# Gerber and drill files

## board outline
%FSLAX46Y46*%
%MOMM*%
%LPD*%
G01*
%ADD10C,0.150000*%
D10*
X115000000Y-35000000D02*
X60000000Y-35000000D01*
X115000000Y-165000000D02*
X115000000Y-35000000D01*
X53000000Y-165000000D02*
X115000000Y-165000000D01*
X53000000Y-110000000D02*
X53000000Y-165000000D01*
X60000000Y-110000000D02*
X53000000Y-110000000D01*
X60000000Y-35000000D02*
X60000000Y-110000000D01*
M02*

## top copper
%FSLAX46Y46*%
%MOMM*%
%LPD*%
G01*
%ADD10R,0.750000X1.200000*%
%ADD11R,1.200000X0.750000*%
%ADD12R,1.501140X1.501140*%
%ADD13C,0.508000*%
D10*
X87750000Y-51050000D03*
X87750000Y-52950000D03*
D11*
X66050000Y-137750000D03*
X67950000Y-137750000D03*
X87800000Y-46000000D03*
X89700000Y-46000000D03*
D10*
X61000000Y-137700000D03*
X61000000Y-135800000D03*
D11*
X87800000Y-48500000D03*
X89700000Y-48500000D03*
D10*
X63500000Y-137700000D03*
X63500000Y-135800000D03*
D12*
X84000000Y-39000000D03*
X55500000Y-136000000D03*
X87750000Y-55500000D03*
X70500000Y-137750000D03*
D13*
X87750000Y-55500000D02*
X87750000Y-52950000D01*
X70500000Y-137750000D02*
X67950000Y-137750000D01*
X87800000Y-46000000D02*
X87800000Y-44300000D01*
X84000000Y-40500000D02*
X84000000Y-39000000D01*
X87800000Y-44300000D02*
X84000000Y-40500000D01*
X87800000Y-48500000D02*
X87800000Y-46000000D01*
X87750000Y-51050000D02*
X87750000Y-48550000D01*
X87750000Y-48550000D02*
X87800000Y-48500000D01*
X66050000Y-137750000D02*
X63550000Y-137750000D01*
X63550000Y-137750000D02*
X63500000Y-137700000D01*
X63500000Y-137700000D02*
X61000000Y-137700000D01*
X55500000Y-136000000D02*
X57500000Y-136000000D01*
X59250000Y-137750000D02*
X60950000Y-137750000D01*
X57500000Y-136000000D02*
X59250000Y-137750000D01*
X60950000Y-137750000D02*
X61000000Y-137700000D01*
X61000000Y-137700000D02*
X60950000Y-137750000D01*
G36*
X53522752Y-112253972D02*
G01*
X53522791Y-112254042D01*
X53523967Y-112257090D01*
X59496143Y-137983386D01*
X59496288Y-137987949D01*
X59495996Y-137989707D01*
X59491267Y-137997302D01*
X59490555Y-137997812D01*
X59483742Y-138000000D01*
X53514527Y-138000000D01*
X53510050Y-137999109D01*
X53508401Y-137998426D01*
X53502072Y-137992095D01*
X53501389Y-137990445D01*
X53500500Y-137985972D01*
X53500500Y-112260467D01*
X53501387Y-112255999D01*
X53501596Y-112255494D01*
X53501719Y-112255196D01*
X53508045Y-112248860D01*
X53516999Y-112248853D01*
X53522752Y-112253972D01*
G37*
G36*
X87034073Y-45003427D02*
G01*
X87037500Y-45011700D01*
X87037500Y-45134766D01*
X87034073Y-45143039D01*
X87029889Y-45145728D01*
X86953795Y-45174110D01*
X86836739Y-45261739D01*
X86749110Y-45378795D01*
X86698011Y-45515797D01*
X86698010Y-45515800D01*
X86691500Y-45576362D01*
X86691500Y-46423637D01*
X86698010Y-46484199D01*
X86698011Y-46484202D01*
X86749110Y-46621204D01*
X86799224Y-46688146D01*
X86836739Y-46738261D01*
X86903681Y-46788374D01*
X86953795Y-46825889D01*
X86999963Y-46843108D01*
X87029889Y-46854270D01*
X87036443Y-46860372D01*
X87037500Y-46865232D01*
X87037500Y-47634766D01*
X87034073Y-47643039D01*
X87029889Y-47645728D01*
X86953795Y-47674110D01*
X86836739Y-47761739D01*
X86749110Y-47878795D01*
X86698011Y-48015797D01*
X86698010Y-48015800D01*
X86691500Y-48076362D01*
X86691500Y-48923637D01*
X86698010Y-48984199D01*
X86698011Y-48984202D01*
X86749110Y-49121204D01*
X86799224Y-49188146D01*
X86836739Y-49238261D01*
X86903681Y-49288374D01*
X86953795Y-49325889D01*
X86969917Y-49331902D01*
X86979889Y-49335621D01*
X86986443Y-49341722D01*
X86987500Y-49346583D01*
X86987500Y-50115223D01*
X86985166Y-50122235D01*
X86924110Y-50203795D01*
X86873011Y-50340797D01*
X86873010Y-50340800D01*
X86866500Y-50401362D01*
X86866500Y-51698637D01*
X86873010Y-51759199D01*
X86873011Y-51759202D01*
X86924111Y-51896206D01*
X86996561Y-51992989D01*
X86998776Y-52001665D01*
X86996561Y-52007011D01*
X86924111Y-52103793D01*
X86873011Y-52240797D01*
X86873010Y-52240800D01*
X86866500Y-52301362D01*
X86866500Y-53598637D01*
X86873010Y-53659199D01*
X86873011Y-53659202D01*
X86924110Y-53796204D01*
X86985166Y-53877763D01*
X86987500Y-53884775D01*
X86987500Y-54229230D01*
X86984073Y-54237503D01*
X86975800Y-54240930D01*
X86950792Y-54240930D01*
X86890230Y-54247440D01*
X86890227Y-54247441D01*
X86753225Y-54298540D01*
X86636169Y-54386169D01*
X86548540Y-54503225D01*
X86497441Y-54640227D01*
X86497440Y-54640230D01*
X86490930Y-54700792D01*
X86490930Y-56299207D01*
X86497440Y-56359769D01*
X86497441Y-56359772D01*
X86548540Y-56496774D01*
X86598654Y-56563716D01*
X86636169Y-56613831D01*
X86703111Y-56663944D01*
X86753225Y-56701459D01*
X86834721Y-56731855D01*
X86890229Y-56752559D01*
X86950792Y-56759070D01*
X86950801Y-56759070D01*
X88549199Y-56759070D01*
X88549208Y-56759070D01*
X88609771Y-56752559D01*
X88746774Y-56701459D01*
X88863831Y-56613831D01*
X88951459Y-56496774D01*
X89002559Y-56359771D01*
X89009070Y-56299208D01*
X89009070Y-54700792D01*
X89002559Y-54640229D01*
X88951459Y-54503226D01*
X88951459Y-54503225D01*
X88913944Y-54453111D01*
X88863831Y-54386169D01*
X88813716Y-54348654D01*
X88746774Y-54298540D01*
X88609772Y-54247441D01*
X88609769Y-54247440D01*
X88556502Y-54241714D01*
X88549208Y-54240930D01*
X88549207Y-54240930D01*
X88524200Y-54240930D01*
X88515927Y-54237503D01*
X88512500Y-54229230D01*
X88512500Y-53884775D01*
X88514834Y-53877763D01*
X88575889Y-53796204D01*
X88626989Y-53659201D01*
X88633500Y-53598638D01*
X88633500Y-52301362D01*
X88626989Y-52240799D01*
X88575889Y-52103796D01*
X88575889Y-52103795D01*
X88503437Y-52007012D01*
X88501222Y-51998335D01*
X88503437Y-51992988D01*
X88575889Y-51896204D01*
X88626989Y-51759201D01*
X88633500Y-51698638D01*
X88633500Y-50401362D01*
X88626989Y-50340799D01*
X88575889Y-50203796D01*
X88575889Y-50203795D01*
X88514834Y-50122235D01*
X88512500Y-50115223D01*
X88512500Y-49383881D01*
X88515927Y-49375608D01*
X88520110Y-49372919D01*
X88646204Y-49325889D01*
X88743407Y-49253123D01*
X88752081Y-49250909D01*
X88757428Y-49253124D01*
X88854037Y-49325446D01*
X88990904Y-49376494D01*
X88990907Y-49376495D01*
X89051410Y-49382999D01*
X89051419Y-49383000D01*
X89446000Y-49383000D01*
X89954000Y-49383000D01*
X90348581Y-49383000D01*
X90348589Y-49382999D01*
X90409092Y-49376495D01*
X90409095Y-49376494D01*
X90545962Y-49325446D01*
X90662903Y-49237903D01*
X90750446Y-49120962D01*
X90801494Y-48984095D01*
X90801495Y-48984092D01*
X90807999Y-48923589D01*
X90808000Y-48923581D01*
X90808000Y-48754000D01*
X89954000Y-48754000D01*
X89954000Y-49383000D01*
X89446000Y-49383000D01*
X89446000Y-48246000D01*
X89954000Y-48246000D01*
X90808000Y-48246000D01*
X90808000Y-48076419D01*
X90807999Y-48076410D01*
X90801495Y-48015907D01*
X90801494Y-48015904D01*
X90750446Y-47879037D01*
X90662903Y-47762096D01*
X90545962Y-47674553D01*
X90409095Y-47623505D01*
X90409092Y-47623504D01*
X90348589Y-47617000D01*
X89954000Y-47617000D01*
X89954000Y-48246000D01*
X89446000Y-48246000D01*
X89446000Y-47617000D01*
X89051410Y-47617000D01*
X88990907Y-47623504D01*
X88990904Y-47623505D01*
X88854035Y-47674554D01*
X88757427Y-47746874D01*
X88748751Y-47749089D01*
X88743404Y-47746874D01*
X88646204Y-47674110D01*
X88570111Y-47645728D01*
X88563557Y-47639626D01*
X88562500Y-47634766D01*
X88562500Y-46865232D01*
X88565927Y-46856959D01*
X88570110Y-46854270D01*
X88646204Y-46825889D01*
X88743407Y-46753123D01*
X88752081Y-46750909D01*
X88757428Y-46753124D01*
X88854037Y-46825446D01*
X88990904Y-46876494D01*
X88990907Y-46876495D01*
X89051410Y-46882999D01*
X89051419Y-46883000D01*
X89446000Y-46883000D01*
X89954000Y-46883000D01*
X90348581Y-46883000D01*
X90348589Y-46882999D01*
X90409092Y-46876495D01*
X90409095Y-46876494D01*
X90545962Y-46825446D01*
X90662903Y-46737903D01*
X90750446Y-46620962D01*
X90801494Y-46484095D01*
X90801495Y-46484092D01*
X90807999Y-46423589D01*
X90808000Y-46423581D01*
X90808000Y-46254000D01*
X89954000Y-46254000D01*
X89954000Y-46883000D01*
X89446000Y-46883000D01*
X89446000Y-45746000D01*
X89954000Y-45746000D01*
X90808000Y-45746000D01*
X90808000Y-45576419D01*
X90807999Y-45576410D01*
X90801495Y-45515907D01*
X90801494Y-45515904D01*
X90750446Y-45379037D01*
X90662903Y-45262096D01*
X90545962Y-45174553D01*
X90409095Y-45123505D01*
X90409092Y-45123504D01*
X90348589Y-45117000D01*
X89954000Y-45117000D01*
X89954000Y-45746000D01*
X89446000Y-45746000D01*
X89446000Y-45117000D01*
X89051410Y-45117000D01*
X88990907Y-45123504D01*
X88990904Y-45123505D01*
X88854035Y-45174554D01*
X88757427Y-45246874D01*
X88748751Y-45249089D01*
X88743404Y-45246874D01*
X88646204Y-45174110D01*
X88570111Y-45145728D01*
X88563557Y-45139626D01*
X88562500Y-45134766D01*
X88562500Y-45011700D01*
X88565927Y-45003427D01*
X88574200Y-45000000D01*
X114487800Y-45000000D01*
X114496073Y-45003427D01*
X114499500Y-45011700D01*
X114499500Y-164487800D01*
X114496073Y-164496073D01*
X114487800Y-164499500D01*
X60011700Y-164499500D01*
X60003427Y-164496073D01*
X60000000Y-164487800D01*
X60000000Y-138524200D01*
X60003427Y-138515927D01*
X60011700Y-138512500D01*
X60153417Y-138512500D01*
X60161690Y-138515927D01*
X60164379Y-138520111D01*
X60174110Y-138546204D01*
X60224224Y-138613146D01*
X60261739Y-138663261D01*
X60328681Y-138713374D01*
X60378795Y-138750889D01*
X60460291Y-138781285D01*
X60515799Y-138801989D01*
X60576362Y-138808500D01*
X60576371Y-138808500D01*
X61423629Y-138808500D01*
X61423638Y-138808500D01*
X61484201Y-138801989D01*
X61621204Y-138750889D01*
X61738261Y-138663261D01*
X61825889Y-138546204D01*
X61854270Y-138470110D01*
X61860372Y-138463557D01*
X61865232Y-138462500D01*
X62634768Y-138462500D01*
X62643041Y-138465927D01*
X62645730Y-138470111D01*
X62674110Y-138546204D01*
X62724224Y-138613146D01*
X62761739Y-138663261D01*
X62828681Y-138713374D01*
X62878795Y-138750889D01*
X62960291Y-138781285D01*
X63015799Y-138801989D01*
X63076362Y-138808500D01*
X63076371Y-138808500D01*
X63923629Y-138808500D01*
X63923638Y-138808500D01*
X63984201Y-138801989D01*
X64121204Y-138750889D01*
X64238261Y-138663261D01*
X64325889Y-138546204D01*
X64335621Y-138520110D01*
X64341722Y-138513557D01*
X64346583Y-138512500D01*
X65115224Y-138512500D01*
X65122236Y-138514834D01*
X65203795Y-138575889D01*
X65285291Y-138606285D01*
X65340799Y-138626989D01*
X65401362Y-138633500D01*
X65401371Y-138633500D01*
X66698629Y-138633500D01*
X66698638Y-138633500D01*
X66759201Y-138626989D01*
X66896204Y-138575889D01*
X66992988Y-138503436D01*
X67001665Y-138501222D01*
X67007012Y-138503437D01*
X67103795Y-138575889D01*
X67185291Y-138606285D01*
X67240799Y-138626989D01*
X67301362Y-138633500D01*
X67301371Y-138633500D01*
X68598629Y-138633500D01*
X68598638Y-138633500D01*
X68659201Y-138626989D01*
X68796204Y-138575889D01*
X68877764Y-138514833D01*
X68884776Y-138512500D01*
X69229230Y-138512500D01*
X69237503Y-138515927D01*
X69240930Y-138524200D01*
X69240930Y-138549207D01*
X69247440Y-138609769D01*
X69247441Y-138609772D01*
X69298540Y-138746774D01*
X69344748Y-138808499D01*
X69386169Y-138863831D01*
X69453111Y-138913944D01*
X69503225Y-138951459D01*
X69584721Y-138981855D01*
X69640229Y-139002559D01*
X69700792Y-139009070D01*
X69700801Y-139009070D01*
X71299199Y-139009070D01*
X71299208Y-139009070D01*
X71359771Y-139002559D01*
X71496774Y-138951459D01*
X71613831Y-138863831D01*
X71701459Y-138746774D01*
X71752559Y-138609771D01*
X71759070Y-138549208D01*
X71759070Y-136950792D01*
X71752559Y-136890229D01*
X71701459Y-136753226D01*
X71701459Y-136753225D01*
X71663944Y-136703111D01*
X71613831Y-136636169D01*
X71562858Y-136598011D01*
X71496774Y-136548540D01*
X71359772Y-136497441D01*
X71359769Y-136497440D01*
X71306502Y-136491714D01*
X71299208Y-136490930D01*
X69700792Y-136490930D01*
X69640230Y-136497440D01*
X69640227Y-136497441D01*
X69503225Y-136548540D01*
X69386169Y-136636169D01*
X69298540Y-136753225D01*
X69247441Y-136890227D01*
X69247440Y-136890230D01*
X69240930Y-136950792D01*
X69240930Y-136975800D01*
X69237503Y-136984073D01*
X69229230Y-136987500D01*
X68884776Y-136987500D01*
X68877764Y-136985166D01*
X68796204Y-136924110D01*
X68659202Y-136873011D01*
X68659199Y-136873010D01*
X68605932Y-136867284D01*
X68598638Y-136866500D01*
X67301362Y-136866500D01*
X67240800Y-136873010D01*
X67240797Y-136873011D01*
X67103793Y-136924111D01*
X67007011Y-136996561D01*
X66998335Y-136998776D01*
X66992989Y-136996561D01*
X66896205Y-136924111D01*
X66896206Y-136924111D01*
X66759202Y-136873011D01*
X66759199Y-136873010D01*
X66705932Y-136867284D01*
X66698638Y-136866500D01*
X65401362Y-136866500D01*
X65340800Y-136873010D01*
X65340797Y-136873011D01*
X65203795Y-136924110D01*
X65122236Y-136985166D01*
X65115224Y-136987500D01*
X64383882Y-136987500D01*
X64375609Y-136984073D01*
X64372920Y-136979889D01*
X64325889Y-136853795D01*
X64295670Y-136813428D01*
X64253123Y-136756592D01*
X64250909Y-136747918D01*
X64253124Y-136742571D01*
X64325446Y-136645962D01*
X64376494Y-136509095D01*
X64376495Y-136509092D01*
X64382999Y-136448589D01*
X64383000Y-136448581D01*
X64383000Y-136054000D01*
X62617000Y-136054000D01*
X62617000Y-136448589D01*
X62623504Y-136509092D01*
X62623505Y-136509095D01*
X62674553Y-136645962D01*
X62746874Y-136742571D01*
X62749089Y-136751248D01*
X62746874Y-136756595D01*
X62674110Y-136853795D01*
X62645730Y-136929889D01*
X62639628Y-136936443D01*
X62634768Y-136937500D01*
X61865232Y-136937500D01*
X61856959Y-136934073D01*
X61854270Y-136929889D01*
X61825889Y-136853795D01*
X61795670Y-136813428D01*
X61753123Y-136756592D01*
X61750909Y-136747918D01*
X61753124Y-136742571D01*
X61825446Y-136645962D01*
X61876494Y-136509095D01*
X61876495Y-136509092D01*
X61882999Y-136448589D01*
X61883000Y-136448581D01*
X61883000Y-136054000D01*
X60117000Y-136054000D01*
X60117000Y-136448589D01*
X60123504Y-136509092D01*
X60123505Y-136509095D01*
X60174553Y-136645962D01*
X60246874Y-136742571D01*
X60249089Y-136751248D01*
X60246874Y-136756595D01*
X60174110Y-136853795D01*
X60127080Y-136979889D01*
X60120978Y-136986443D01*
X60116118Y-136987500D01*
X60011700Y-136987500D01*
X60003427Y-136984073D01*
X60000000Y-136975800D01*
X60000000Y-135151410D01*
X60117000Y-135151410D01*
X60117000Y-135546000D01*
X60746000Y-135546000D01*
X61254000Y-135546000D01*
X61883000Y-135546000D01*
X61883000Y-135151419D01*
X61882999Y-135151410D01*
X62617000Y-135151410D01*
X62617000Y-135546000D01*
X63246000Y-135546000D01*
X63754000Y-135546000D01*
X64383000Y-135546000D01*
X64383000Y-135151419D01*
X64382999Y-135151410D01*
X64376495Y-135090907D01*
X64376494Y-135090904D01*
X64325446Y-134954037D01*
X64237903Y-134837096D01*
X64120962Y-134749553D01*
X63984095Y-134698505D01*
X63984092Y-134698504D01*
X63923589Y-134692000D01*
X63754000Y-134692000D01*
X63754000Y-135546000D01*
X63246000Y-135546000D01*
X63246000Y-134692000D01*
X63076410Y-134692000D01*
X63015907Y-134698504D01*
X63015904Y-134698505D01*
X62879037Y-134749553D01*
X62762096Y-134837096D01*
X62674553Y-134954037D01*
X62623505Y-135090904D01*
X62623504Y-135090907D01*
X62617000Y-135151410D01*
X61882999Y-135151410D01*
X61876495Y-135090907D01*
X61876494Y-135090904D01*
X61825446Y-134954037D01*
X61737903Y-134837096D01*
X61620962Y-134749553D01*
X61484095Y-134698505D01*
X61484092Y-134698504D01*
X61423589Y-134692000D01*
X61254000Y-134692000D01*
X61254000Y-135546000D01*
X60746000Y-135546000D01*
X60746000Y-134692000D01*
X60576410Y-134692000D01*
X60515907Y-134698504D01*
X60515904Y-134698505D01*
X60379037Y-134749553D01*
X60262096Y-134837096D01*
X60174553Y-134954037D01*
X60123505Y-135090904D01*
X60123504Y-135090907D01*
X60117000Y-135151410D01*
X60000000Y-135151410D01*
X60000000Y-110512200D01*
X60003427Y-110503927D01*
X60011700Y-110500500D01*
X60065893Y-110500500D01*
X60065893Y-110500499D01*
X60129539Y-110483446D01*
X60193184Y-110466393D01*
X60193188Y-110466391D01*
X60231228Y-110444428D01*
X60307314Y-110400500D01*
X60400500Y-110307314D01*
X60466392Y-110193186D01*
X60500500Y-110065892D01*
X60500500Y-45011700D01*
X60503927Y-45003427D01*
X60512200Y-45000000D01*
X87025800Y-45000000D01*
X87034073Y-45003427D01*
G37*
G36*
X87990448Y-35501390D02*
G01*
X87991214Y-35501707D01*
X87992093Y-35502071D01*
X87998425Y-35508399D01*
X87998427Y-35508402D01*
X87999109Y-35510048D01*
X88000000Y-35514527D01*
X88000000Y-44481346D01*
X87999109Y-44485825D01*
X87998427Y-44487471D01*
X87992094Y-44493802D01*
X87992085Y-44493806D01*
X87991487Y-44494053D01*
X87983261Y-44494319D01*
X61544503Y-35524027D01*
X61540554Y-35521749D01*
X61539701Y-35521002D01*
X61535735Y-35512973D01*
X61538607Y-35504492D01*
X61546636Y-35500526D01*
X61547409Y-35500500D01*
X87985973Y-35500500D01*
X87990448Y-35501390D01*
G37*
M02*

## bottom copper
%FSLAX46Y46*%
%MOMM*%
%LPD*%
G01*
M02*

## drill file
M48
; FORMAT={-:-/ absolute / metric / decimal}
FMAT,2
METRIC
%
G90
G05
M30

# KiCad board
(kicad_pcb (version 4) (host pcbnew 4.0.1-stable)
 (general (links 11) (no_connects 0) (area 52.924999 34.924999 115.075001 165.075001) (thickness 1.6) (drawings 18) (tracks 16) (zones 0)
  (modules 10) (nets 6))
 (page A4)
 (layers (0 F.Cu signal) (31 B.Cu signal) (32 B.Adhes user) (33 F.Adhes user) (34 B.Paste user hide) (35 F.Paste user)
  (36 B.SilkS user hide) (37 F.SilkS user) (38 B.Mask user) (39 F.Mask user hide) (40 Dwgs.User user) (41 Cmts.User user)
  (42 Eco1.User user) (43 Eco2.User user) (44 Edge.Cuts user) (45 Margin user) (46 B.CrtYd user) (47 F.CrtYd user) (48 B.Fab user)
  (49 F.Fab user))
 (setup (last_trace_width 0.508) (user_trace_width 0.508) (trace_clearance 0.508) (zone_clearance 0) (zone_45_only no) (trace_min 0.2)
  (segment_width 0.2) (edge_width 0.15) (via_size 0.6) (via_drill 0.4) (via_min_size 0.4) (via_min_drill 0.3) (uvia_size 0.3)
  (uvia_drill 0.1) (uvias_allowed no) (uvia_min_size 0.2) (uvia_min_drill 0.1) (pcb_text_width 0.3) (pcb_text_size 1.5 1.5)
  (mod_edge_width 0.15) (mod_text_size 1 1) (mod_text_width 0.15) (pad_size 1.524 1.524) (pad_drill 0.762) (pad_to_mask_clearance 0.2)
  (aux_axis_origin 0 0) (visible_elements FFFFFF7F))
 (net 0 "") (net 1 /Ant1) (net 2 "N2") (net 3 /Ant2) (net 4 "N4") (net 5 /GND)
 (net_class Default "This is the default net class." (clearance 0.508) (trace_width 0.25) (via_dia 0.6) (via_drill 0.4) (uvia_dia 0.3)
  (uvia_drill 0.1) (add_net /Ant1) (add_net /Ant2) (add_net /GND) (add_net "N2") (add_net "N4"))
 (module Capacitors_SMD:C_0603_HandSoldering (layer F.Cu) (at 87.75 52 270)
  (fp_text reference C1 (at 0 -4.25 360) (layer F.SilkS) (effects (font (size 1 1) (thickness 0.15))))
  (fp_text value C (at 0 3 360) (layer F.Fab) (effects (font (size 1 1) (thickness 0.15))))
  (pad 1 smd rect (at -0.95 0 270) (size 1.2 0.75) (layers F.Cu F.Paste F.Mask) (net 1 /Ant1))
  (pad 2 smd rect (at 0.95 0 270) (size 1.2 0.75) (layers F.Cu F.Paste F.Mask) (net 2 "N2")))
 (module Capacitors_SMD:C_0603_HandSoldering (layer F.Cu) (at 67 137.75)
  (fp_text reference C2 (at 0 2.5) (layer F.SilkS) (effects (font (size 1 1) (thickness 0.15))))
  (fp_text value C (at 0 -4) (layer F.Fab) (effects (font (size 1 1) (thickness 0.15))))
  (pad 1 smd rect (at -0.95 0) (size 1.2 0.75) (layers F.Cu F.Paste F.Mask) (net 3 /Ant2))
  (pad 2 smd rect (at 0.95 0) (size 1.2 0.75) (layers F.Cu F.Paste F.Mask) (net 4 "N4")))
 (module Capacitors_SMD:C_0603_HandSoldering (layer F.Cu) (at 88.75 46)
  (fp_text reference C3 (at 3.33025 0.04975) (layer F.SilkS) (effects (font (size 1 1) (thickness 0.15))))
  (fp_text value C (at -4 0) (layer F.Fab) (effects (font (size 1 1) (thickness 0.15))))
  (pad 1 smd rect (at -0.95 0) (size 1.2 0.75) (layers F.Cu F.Paste F.Mask) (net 1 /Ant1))
  (pad 2 smd rect (at 0.95 0) (size 1.2 0.75) (layers F.Cu F.Paste F.Mask) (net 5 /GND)))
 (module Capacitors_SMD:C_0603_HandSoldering (layer F.Cu) (at 61 136.75 90)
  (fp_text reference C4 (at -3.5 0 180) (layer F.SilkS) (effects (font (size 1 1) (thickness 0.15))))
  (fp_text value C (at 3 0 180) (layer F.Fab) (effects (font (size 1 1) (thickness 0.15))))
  (pad 1 smd rect (at -0.95 0 90) (size 1.2 0.75) (layers F.Cu F.Paste F.Mask) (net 3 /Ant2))
  (pad 2 smd rect (at 0.95 0 90) (size 1.2 0.75) (layers F.Cu F.Paste F.Mask) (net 5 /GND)))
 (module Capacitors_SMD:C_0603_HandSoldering (layer F.Cu) (at 88.75 48.5)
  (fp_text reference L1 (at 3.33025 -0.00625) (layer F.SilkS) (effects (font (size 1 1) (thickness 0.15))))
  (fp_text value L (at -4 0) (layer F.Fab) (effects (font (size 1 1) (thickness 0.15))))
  (pad 1 smd rect (at -0.95 0) (size 1.2 0.75) (layers F.Cu F.Paste F.Mask) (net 1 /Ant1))
  (pad 2 smd rect (at 0.95 0) (size 1.2 0.75) (layers F.Cu F.Paste F.Mask) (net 5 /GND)))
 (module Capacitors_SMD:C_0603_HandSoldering (layer F.Cu) (at 63.5 136.75 90)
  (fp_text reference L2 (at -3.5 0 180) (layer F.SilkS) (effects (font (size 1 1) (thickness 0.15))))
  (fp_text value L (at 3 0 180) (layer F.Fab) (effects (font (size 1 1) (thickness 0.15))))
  (pad 1 smd rect (at -0.95 0 90) (size 1.2 0.75) (layers F.Cu F.Paste F.Mask) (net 3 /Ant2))
  (pad 2 smd rect (at 0.95 0 90) (size 1.2 0.75) (layers F.Cu F.Paste F.Mask) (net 5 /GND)))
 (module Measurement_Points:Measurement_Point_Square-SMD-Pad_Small (layer F.Cu) (at 84 39)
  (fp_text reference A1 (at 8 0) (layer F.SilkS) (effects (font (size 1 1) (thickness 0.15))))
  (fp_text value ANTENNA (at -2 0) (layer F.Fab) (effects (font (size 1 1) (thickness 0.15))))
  (pad 1 smd rect (at 0 0) (size 1.50114 1.50114) (layers F.Cu F.Paste F.Mask) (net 1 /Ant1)))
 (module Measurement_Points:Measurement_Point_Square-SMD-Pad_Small (layer F.Cu) (at 55.5 136)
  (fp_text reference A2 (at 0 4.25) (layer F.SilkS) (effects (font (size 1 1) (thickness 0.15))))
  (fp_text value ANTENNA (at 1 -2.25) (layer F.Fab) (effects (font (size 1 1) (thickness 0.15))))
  (pad 1 smd rect (at 0 0) (size 1.50114 1.50114) (layers F.Cu F.Paste F.Mask) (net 3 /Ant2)))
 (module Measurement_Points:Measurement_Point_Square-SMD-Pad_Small (layer F.Cu) (at 87.75 55.5 90)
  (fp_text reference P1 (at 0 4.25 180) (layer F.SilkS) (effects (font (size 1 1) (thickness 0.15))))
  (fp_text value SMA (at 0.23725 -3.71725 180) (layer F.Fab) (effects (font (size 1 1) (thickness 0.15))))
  (pad 1 smd rect (at 0 0 90) (size 1.50114 1.50114) (layers F.Cu F.Paste F.Mask) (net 2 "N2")))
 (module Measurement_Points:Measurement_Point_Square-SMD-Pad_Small (layer F.Cu) (at 70.5 137.75 180)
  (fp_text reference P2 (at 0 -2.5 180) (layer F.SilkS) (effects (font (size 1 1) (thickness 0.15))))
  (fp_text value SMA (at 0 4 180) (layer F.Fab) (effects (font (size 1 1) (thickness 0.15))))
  (pad 1 smd rect (at 0 0 180) (size 1.50114 1.50114) (layers F.Cu F.Paste F.Mask) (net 4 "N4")))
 (gr_line (start 115 35) (end 60 35) (angle 90) (layer Edge.Cuts) (width 0.15))
 (gr_line (start 115 165) (end 115 35) (angle 90) (layer Edge.Cuts) (width 0.15))
 (gr_line (start 53 165) (end 115 165) (angle 90) (layer Edge.Cuts) (width 0.15))
 (gr_line (start 53 110) (end 53 165) (angle 90) (layer Edge.Cuts) (width 0.15))
 (gr_line (start 60 110) (end 53 110) (angle 90) (layer Edge.Cuts) (width 0.15))
 (gr_line (start 60 35) (end 60 110) (angle 90) (layer Edge.Cuts) (width 0.15))
 (segment (start 87.75 55.5) (end 87.75 52.95) (width 0.508) (layer F.Cu) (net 2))
 (segment (start 70.5 137.75) (end 67.95 137.75) (width 0.508) (layer F.Cu) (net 4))
 (segment (start 87.8 46) (end 87.8 44.3) (width 0.508) (layer F.Cu) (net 1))
 (segment (start 84 40.5) (end 84 39) (width 0.508) (layer F.Cu) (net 1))
 (segment (start 87.8 44.3) (end 84 40.5) (width 0.508) (layer F.Cu) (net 1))
 (segment (start 87.8 48.5) (end 87.8 46) (width 0.508) (layer F.Cu) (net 1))
 (segment (start 87.75 51.05) (end 87.75 48.55) (width 0.508) (layer F.Cu) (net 1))
 (segment (start 87.75 48.55) (end 87.8 48.5) (width 0.508) (layer F.Cu) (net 1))
 (segment (start 66.05 137.75) (end 63.55 137.75) (width 0.508) (layer F.Cu) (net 3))
 (segment (start 63.55 137.75) (end 63.5 137.7) (width 0.508) (layer F.Cu) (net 3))
 (segment (start 63.5 137.7) (end 61 137.7) (width 0.508) (layer F.Cu) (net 3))
 (segment (start 55.5 136) (end 57.5 136) (width 0.508) (layer F.Cu) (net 3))
 (segment (start 59.25 137.75) (end 60.95 137.75) (width 0.508) (layer F.Cu) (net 3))
 (segment (start 57.5 136) (end 59.25 137.75) (width 0.508) (layer F.Cu) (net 3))
 (segment (start 60.95 137.75) (end 61 137.7) (width 0.508) (layer F.Cu) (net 3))
 (segment (start 61 137.7) (end 60.95 137.75) (width 0.508) (layer F.Cu) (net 3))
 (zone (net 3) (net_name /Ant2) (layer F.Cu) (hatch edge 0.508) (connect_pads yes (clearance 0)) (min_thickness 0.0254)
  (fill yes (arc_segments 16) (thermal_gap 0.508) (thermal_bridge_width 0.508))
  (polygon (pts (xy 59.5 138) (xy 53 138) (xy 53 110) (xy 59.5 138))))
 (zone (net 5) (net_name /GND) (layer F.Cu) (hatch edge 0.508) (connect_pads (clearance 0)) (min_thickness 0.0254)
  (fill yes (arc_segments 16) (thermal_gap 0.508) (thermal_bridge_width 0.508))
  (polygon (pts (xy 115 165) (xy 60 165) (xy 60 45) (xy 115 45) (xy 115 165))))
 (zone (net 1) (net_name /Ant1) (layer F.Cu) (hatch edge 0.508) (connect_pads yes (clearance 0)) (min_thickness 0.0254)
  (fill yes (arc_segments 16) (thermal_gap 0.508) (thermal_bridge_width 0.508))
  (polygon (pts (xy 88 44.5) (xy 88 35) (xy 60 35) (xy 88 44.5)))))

